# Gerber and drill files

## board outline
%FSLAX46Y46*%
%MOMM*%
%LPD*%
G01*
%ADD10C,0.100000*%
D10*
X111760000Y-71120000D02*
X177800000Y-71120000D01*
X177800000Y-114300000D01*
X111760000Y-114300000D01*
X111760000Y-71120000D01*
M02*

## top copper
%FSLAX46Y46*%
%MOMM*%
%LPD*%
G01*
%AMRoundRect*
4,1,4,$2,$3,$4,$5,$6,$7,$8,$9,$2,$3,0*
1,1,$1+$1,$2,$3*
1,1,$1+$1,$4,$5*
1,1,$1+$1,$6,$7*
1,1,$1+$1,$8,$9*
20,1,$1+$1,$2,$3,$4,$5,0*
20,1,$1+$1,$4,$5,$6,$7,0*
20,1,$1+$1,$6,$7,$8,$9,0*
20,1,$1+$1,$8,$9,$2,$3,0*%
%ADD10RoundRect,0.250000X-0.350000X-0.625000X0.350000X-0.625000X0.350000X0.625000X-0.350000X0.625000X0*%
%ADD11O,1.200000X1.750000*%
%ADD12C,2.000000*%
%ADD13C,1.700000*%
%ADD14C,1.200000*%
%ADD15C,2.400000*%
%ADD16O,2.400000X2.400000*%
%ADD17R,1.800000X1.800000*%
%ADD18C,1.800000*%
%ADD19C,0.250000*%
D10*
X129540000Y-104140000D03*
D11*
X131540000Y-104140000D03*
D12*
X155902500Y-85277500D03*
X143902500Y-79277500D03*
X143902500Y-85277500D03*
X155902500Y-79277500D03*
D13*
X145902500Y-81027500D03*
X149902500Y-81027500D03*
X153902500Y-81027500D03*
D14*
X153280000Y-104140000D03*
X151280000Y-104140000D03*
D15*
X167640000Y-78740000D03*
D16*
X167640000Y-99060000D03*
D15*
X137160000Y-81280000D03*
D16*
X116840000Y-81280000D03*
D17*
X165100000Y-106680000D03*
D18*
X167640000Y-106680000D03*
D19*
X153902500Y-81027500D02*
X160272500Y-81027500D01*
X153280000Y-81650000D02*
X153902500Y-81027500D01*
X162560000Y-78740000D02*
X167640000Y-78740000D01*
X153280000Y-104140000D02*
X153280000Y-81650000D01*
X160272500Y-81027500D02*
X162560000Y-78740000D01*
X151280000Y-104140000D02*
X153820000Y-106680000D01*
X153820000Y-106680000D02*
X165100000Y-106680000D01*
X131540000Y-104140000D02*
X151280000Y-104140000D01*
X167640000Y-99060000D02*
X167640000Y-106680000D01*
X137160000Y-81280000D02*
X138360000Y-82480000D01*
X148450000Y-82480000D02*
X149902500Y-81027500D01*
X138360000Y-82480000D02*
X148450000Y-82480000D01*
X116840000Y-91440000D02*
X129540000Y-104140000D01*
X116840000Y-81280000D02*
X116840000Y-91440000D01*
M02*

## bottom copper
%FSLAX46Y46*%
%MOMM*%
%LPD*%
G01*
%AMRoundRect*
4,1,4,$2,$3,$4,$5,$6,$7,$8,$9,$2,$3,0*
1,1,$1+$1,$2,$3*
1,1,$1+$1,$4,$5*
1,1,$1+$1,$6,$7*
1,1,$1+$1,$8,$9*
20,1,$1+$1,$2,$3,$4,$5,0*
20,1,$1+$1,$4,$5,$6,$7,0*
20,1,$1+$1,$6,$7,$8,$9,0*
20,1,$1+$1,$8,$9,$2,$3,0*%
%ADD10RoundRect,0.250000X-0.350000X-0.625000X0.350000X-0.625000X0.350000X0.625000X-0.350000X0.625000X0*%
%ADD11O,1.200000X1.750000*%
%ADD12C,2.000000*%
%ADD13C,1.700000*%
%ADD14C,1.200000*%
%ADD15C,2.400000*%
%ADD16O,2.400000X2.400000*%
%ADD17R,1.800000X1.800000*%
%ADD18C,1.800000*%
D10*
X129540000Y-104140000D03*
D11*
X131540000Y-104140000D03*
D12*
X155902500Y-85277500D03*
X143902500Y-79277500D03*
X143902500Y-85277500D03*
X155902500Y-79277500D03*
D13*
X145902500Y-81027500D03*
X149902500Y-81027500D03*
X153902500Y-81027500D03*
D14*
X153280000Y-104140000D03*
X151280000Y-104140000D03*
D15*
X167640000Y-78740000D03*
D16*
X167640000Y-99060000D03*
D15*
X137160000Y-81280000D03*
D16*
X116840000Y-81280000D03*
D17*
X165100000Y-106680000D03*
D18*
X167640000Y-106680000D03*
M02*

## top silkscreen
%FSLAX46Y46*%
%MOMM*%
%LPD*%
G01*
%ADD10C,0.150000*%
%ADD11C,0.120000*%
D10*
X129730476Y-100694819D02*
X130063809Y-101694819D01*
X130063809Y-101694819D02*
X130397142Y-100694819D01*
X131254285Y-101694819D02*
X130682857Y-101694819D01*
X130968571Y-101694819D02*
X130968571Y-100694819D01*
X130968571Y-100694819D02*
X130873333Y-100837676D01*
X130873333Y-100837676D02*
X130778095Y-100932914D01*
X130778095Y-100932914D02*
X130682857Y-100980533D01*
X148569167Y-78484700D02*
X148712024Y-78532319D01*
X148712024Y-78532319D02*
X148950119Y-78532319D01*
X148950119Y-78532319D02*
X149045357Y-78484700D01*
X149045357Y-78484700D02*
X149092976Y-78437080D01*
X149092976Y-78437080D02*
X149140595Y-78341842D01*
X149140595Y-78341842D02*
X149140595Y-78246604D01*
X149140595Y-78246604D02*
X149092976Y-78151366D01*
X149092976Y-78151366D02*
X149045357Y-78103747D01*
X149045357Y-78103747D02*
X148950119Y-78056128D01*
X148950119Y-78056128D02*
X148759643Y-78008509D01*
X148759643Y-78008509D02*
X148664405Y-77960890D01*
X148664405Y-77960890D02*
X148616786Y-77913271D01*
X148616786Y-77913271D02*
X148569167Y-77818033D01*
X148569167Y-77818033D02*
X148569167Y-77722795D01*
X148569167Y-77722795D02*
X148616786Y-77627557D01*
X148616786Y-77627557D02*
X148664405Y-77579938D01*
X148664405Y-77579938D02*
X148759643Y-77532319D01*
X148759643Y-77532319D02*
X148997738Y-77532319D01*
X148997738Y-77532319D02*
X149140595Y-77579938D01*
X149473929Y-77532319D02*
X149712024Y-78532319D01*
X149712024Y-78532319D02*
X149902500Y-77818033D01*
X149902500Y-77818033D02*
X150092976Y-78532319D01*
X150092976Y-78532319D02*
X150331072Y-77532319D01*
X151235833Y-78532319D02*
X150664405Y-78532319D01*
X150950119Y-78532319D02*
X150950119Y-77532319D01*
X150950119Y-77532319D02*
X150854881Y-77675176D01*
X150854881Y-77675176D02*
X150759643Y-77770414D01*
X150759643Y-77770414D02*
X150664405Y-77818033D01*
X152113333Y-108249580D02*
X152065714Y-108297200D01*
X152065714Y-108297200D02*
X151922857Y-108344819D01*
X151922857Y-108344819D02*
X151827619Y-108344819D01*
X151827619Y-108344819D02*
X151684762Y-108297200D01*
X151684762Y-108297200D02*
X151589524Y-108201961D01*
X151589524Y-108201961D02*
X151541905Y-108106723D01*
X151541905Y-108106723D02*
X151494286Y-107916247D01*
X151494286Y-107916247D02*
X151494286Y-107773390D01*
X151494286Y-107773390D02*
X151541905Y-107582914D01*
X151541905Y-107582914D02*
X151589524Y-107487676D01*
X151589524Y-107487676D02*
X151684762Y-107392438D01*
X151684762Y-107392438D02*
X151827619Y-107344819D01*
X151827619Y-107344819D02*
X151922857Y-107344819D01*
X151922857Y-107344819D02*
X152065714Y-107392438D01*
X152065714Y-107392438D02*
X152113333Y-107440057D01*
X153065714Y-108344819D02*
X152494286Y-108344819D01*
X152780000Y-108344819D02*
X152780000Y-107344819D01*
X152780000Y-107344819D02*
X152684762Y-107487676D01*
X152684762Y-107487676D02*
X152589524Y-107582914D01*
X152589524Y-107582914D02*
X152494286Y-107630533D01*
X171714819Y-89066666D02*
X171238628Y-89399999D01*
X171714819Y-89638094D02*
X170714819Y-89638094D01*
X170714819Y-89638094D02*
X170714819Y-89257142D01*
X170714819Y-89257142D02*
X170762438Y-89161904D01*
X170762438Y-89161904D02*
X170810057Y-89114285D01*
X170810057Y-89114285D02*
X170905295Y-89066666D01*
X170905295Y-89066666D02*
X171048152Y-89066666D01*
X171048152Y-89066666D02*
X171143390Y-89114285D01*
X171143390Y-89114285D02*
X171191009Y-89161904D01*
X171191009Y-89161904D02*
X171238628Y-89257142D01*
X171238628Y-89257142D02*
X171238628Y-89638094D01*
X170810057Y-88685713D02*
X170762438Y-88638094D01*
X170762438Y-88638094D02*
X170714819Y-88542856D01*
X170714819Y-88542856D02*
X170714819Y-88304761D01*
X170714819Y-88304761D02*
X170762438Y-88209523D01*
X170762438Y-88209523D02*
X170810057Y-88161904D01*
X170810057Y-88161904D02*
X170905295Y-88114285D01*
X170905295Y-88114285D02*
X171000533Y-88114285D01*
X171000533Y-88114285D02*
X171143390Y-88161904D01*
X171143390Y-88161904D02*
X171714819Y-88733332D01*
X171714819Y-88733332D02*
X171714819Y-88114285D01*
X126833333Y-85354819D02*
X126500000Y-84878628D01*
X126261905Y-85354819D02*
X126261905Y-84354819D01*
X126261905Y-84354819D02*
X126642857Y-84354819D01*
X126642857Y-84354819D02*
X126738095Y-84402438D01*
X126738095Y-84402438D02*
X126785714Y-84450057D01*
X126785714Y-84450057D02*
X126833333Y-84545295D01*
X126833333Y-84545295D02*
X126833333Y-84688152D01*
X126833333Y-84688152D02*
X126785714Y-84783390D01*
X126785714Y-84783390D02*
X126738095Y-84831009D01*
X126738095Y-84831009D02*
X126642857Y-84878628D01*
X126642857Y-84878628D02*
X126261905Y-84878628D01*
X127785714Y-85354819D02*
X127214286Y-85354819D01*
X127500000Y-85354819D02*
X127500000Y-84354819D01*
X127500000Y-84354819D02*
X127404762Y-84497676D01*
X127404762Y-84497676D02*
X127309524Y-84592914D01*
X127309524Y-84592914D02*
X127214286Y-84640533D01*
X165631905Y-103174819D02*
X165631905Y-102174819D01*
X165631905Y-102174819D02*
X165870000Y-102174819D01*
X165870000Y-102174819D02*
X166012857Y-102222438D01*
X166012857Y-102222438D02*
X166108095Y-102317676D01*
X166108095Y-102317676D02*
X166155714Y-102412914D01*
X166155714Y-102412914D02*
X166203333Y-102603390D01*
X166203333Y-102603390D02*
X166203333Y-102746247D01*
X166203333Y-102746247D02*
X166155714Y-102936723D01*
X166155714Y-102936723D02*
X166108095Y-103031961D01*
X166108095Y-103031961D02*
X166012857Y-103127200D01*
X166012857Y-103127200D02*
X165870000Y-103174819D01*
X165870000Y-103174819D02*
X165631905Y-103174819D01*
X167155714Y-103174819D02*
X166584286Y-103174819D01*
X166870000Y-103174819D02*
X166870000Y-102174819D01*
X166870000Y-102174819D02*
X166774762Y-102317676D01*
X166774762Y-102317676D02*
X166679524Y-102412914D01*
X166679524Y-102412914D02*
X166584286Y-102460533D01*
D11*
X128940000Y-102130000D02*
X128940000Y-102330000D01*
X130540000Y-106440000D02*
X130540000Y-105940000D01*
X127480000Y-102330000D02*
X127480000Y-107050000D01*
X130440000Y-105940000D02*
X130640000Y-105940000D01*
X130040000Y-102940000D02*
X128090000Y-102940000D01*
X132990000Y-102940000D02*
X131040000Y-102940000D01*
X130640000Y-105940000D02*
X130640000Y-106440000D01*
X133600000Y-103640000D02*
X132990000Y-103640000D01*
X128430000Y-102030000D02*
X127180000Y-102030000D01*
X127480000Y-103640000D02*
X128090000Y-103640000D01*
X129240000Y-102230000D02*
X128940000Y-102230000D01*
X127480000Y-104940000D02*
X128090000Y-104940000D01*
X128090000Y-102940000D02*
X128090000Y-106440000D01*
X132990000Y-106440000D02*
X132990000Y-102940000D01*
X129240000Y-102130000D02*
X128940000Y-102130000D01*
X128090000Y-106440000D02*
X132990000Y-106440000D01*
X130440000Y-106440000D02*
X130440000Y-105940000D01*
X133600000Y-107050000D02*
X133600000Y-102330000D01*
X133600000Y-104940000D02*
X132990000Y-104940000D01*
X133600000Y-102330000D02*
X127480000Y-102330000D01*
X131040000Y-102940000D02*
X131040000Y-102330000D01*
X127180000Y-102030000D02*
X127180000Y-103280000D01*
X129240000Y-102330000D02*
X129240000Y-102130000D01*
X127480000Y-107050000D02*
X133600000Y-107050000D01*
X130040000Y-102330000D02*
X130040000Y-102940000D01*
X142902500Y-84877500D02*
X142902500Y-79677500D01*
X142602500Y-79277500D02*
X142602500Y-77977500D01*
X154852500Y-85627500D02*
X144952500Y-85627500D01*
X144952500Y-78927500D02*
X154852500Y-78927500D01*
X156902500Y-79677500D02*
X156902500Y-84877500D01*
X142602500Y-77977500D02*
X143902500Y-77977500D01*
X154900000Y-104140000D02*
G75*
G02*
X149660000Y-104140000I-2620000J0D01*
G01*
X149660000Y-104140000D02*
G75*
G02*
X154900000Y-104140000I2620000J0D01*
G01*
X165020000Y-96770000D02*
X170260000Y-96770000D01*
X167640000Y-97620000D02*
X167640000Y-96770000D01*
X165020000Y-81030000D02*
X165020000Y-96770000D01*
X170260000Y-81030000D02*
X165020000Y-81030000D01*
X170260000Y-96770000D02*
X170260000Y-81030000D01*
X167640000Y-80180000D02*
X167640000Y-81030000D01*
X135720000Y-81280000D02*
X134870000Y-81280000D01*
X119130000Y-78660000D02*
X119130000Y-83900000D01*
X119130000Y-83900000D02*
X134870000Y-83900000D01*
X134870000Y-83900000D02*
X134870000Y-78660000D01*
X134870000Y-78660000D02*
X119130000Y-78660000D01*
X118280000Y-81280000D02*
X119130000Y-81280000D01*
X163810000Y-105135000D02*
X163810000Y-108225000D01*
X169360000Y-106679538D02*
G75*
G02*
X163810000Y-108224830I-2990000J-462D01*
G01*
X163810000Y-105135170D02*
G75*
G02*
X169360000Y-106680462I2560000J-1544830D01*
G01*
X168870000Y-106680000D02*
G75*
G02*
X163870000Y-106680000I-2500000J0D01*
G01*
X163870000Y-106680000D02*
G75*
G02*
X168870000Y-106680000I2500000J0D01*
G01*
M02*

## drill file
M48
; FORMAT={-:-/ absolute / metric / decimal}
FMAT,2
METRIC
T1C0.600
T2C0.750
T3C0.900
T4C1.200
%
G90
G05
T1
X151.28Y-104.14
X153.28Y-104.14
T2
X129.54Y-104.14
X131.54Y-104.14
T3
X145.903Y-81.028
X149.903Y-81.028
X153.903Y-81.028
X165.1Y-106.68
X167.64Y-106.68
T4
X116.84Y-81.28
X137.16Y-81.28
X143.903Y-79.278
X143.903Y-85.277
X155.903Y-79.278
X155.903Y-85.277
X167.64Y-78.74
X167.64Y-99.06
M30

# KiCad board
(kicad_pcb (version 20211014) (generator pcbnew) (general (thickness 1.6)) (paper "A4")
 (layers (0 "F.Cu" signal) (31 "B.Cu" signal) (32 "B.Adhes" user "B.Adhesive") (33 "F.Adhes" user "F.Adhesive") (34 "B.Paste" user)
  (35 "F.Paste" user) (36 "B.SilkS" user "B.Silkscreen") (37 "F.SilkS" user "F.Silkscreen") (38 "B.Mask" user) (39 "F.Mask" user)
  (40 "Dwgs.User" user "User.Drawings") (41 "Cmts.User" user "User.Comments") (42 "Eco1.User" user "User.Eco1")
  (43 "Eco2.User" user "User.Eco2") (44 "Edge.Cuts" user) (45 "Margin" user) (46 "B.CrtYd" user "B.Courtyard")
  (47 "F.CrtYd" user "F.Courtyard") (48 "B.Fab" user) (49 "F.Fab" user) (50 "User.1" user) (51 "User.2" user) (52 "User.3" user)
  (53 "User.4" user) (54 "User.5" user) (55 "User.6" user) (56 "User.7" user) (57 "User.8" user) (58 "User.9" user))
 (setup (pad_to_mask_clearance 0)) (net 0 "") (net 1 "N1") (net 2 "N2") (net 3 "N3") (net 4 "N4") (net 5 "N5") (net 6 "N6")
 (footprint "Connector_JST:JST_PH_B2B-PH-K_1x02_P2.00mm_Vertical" (layer "F.Cu") (at 129.54 104.14)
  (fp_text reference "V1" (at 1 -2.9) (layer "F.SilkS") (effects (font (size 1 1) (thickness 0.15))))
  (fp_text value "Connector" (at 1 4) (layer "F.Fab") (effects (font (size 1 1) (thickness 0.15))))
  (fp_line (start -0.6 -2.01) (end -0.6 -1.81) (layer "F.SilkS") (width 0.12))
  (fp_line (start 1 2.3) (end 1 1.8) (layer "F.SilkS") (width 0.12))
  (fp_line (start -2.06 -1.81) (end -2.06 2.91) (layer "F.SilkS") (width 0.12))
  (fp_line (start 0.9 1.8) (end 1.1 1.8) (layer "F.SilkS") (width 0.12))
  (fp_line (start 0.5 -1.2) (end -1.45 -1.2) (layer "F.SilkS") (width 0.12))
  (fp_line (start 3.45 -1.2) (end 1.5 -1.2) (layer "F.SilkS") (width 0.12))
  (fp_line (start 1.1 1.8) (end 1.1 2.3) (layer "F.SilkS") (width 0.12))
  (fp_line (start 4.06 -0.5) (end 3.45 -0.5) (layer "F.SilkS") (width 0.12))
  (fp_line (start -1.11 -2.11) (end -2.36 -2.11) (layer "F.SilkS") (width 0.12))
  (fp_line (start -2.06 -0.5) (end -1.45 -0.5) (layer "F.SilkS") (width 0.12))
  (fp_line (start -0.3 -1.91) (end -0.6 -1.91) (layer "F.SilkS") (width 0.12))
  (fp_line (start -2.06 0.8) (end -1.45 0.8) (layer "F.SilkS") (width 0.12))
  (fp_line (start -1.45 -1.2) (end -1.45 2.3) (layer "F.SilkS") (width 0.12))
  (fp_line (start 3.45 2.3) (end 3.45 -1.2) (layer "F.SilkS") (width 0.12))
  (fp_line (start -0.3 -2.01) (end -0.6 -2.01) (layer "F.SilkS") (width 0.12))
  (fp_line (start -1.45 2.3) (end 3.45 2.3) (layer "F.SilkS") (width 0.12))
  (fp_line (start 0.9 2.3) (end 0.9 1.8) (layer "F.SilkS") (width 0.12))
  (fp_line (start 4.06 2.91) (end 4.06 -1.81) (layer "F.SilkS") (width 0.12))
  (fp_line (start 4.06 0.8) (end 3.45 0.8) (layer "F.SilkS") (width 0.12))
  (fp_line (start 4.06 -1.81) (end -2.06 -1.81) (layer "F.SilkS") (width 0.12))
  (fp_line (start 1.5 -1.2) (end 1.5 -1.81) (layer "F.SilkS") (width 0.12))
  (fp_line (start -2.36 -2.11) (end -2.36 -0.86) (layer "F.SilkS") (width 0.12))
  (fp_line (start -0.3 -1.81) (end -0.3 -2.01) (layer "F.SilkS") (width 0.12))
  (fp_line (start -2.06 2.91) (end 4.06 2.91) (layer "F.SilkS") (width 0.12))
  (fp_line (start 0.5 -1.81) (end 0.5 -1.2) (layer "F.SilkS") (width 0.12))
  (pad "1" thru_hole roundrect (at 0 0) (size 1.2 1.75) (drill 0.75) (layers *.Cu *.Mask) (roundrect_rratio 0.208333) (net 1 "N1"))
  (pad "2" thru_hole oval (at 2 0) (size 1.2 1.75) (drill 0.75) (layers *.Cu *.Mask) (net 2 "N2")))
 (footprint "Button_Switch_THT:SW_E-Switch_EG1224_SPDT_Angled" (layer "F.Cu") (at 145.9025 81.0275)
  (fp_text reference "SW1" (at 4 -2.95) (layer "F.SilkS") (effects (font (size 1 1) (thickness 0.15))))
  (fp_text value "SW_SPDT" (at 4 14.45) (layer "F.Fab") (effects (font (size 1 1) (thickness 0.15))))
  (fp_line (start -3 3.85) (end -3 -1.35) (layer "F.SilkS") (width 0.12))
  (fp_line (start -3.3 -1.75) (end -3.3 -3.05) (layer "F.SilkS") (width 0.12))
  (fp_line (start 8.95 4.6) (end -0.95 4.6) (layer "F.SilkS") (width 0.12))
  (fp_line (start -0.95 -2.1) (end 8.95 -2.1) (layer "F.SilkS") (width 0.12))
  (fp_line (start 11 -1.35) (end 11 3.85) (layer "F.SilkS") (width 0.12))
  (fp_line (start -3.3 -3.05) (end -2 -3.05) (layer "F.SilkS") (width 0.12))
  (pad "" thru_hole circle (at 10 4.25) (size 2 2) (drill 1.2) (layers *.Cu *.Mask))
  (pad "" thru_hole circle (at -2 -1.75) (size 2 2) (drill 1.2) (layers *.Cu *.Mask))
  (pad "" thru_hole circle (at -2 4.25) (size 2 2) (drill 1.2) (layers *.Cu *.Mask))
  (pad "" thru_hole circle (at 10 -1.75) (size 2 2) (drill 1.2) (layers *.Cu *.Mask))
  (pad "1" thru_hole circle (at 0 0) (size 1.7 1.7) (drill 0.9) (layers *.Cu *.Mask) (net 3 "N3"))
  (pad "2" thru_hole circle (at 4 0) (size 1.7 1.7) (drill 0.9) (layers *.Cu *.Mask) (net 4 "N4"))
  (pad "3" thru_hole circle (at 8 0) (size 1.7 1.7) (drill 0.9) (layers *.Cu *.Mask) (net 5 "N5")))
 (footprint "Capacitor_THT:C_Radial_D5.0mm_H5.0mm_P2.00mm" (layer "F.Cu") (at 153.28 104.14 180)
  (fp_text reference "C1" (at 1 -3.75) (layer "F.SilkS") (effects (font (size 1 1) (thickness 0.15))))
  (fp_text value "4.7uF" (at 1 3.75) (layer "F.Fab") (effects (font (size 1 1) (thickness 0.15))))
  (fp_circle (center 1 0) (end 3.62 0) (layer "F.SilkS") (width 0.12) (fill none))
  (pad "1" thru_hole circle (at 0 0 180) (size 1.2 1.2) (drill 0.6) (layers *.Cu *.Mask) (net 5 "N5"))
  (pad "2" thru_hole circle (at 2 0 180) (size 1.2 1.2) (drill 0.6) (layers *.Cu *.Mask) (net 2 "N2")))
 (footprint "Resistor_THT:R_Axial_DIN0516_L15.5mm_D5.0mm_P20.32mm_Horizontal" (layer "F.Cu") (at 167.64 78.74 -90)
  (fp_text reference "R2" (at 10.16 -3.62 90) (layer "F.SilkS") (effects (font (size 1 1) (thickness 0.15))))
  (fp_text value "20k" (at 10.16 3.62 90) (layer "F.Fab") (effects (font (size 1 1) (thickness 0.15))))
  (fp_line (start 18.03 2.62) (end 18.03 -2.62) (layer "F.SilkS") (width 0.12))
  (fp_line (start 18.88 0) (end 18.03 0) (layer "F.SilkS") (width 0.12))
  (fp_line (start 2.29 2.62) (end 18.03 2.62) (layer "F.SilkS") (width 0.12))
  (fp_line (start 2.29 -2.62) (end 2.29 2.62) (layer "F.SilkS") (width 0.12))
  (fp_line (start 18.03 -2.62) (end 2.29 -2.62) (layer "F.SilkS") (width 0.12))
  (fp_line (start 1.44 0) (end 2.29 0) (layer "F.SilkS") (width 0.12))
  (pad "1" thru_hole circle (at 0 0 270) (size 2.4 2.4) (drill 1.2) (layers *.Cu *.Mask) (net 5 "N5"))
  (pad "2" thru_hole oval (at 20.32 0 270) (size 2.4 2.4) (drill 1.2) (layers *.Cu *.Mask) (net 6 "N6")))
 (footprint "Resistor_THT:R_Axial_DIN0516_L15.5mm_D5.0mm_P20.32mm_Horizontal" (layer "F.Cu") (at 137.16 81.28 180)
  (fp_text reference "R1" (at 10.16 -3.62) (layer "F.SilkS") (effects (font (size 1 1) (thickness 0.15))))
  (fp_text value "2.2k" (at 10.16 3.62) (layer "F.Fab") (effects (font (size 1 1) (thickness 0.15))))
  (fp_line (start 1.44 0) (end 2.29 0) (layer "F.SilkS") (width 0.12))
  (fp_line (start 18.03 2.62) (end 18.03 -2.62) (layer "F.SilkS") (width 0.12))
  (fp_line (start 18.03 -2.62) (end 2.29 -2.62) (layer "F.SilkS") (width 0.12))
  (fp_line (start 2.29 -2.62) (end 2.29 2.62) (layer "F.SilkS") (width 0.12))
  (fp_line (start 2.29 2.62) (end 18.03 2.62) (layer "F.SilkS") (width 0.12))
  (fp_line (start 18.88 0) (end 18.03 0) (layer "F.SilkS") (width 0.12))
  (pad "1" thru_hole circle (at 0 0 180) (size 2.4 2.4) (drill 1.2) (layers *.Cu *.Mask) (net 4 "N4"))
  (pad "2" thru_hole oval (at 20.32 0 180) (size 2.4 2.4) (drill 1.2) (layers *.Cu *.Mask) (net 1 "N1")))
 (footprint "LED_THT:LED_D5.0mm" (layer "F.Cu") (at 165.1 106.68)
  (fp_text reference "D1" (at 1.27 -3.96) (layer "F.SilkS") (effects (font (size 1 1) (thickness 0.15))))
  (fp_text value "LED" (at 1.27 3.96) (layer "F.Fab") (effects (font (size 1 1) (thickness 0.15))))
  (fp_line (start -1.29 -1.545) (end -1.29 1.545) (layer "F.SilkS") (width 0.12))
  (fp_arc (start 4.26 -0.000462) (mid 2.072002 2.880433) (end -1.29 1.54483) (layer "F.SilkS") (width 0.12))
  (fp_arc (start -1.29 -1.54483) (mid 2.072002 -2.880433) (end 4.26 0.000462) (layer "F.SilkS") (width 0.12))
  (fp_circle (center 1.27 0) (end 3.77 0) (layer "F.SilkS") (width 0.12) (fill none))
  (pad "1" thru_hole rect (at 0 0) (size 1.8 1.8) (drill 0.9) (layers *.Cu *.Mask) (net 2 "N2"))
  (pad "2" thru_hole circle (at 2.54 0) (size 1.8 1.8) (drill 0.9) (layers *.Cu *.Mask) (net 6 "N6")))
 (gr_rect (start 111.76 71.12) (end 177.8 114.3) (layer "Edge.Cuts") (width 0.1) (fill none))
 (segment (start 153.9025 81.0275) (end 160.2725 81.0275) (width 0.25) (layer "F.Cu") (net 5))
 (segment (start 153.28 81.65) (end 153.9025 81.0275) (width 0.25) (layer "F.Cu") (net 5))
 (segment (start 162.56 78.74) (end 167.64 78.74) (width 0.25) (layer "F.Cu") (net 5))
 (segment (start 153.28 104.14) (end 153.28 81.65) (width 0.25) (layer "F.Cu") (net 5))
 (segment (start 160.2725 81.0275) (end 162.56 78.74) (width 0.25) (layer "F.Cu") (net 5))
 (segment (start 151.28 104.14) (end 153.82 106.68) (width 0.25) (layer "F.Cu") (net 2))
 (segment (start 153.82 106.68) (end 165.1 106.68) (width 0.25) (layer "F.Cu") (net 2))
 (segment (start 131.54 104.14) (end 151.28 104.14) (width 0.25) (layer "F.Cu") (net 2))
 (segment (start 167.64 99.06) (end 167.64 106.68) (width 0.25) (layer "F.Cu") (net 6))
 (segment (start 137.16 81.28) (end 138.36 82.48) (width 0.25) (layer "F.Cu") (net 4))
 (segment (start 148.45 82.48) (end 149.9025 81.0275) (width 0.25) (layer "F.Cu") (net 4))
 (segment (start 138.36 82.48) (end 148.45 82.48) (width 0.25) (layer "F.Cu") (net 4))
 (segment (start 116.84 91.44) (end 129.54 104.14) (width 0.25) (layer "F.Cu") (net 1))
 (segment (start 116.84 81.28) (end 116.84 91.44) (width 0.25) (layer "F.Cu") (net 1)))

